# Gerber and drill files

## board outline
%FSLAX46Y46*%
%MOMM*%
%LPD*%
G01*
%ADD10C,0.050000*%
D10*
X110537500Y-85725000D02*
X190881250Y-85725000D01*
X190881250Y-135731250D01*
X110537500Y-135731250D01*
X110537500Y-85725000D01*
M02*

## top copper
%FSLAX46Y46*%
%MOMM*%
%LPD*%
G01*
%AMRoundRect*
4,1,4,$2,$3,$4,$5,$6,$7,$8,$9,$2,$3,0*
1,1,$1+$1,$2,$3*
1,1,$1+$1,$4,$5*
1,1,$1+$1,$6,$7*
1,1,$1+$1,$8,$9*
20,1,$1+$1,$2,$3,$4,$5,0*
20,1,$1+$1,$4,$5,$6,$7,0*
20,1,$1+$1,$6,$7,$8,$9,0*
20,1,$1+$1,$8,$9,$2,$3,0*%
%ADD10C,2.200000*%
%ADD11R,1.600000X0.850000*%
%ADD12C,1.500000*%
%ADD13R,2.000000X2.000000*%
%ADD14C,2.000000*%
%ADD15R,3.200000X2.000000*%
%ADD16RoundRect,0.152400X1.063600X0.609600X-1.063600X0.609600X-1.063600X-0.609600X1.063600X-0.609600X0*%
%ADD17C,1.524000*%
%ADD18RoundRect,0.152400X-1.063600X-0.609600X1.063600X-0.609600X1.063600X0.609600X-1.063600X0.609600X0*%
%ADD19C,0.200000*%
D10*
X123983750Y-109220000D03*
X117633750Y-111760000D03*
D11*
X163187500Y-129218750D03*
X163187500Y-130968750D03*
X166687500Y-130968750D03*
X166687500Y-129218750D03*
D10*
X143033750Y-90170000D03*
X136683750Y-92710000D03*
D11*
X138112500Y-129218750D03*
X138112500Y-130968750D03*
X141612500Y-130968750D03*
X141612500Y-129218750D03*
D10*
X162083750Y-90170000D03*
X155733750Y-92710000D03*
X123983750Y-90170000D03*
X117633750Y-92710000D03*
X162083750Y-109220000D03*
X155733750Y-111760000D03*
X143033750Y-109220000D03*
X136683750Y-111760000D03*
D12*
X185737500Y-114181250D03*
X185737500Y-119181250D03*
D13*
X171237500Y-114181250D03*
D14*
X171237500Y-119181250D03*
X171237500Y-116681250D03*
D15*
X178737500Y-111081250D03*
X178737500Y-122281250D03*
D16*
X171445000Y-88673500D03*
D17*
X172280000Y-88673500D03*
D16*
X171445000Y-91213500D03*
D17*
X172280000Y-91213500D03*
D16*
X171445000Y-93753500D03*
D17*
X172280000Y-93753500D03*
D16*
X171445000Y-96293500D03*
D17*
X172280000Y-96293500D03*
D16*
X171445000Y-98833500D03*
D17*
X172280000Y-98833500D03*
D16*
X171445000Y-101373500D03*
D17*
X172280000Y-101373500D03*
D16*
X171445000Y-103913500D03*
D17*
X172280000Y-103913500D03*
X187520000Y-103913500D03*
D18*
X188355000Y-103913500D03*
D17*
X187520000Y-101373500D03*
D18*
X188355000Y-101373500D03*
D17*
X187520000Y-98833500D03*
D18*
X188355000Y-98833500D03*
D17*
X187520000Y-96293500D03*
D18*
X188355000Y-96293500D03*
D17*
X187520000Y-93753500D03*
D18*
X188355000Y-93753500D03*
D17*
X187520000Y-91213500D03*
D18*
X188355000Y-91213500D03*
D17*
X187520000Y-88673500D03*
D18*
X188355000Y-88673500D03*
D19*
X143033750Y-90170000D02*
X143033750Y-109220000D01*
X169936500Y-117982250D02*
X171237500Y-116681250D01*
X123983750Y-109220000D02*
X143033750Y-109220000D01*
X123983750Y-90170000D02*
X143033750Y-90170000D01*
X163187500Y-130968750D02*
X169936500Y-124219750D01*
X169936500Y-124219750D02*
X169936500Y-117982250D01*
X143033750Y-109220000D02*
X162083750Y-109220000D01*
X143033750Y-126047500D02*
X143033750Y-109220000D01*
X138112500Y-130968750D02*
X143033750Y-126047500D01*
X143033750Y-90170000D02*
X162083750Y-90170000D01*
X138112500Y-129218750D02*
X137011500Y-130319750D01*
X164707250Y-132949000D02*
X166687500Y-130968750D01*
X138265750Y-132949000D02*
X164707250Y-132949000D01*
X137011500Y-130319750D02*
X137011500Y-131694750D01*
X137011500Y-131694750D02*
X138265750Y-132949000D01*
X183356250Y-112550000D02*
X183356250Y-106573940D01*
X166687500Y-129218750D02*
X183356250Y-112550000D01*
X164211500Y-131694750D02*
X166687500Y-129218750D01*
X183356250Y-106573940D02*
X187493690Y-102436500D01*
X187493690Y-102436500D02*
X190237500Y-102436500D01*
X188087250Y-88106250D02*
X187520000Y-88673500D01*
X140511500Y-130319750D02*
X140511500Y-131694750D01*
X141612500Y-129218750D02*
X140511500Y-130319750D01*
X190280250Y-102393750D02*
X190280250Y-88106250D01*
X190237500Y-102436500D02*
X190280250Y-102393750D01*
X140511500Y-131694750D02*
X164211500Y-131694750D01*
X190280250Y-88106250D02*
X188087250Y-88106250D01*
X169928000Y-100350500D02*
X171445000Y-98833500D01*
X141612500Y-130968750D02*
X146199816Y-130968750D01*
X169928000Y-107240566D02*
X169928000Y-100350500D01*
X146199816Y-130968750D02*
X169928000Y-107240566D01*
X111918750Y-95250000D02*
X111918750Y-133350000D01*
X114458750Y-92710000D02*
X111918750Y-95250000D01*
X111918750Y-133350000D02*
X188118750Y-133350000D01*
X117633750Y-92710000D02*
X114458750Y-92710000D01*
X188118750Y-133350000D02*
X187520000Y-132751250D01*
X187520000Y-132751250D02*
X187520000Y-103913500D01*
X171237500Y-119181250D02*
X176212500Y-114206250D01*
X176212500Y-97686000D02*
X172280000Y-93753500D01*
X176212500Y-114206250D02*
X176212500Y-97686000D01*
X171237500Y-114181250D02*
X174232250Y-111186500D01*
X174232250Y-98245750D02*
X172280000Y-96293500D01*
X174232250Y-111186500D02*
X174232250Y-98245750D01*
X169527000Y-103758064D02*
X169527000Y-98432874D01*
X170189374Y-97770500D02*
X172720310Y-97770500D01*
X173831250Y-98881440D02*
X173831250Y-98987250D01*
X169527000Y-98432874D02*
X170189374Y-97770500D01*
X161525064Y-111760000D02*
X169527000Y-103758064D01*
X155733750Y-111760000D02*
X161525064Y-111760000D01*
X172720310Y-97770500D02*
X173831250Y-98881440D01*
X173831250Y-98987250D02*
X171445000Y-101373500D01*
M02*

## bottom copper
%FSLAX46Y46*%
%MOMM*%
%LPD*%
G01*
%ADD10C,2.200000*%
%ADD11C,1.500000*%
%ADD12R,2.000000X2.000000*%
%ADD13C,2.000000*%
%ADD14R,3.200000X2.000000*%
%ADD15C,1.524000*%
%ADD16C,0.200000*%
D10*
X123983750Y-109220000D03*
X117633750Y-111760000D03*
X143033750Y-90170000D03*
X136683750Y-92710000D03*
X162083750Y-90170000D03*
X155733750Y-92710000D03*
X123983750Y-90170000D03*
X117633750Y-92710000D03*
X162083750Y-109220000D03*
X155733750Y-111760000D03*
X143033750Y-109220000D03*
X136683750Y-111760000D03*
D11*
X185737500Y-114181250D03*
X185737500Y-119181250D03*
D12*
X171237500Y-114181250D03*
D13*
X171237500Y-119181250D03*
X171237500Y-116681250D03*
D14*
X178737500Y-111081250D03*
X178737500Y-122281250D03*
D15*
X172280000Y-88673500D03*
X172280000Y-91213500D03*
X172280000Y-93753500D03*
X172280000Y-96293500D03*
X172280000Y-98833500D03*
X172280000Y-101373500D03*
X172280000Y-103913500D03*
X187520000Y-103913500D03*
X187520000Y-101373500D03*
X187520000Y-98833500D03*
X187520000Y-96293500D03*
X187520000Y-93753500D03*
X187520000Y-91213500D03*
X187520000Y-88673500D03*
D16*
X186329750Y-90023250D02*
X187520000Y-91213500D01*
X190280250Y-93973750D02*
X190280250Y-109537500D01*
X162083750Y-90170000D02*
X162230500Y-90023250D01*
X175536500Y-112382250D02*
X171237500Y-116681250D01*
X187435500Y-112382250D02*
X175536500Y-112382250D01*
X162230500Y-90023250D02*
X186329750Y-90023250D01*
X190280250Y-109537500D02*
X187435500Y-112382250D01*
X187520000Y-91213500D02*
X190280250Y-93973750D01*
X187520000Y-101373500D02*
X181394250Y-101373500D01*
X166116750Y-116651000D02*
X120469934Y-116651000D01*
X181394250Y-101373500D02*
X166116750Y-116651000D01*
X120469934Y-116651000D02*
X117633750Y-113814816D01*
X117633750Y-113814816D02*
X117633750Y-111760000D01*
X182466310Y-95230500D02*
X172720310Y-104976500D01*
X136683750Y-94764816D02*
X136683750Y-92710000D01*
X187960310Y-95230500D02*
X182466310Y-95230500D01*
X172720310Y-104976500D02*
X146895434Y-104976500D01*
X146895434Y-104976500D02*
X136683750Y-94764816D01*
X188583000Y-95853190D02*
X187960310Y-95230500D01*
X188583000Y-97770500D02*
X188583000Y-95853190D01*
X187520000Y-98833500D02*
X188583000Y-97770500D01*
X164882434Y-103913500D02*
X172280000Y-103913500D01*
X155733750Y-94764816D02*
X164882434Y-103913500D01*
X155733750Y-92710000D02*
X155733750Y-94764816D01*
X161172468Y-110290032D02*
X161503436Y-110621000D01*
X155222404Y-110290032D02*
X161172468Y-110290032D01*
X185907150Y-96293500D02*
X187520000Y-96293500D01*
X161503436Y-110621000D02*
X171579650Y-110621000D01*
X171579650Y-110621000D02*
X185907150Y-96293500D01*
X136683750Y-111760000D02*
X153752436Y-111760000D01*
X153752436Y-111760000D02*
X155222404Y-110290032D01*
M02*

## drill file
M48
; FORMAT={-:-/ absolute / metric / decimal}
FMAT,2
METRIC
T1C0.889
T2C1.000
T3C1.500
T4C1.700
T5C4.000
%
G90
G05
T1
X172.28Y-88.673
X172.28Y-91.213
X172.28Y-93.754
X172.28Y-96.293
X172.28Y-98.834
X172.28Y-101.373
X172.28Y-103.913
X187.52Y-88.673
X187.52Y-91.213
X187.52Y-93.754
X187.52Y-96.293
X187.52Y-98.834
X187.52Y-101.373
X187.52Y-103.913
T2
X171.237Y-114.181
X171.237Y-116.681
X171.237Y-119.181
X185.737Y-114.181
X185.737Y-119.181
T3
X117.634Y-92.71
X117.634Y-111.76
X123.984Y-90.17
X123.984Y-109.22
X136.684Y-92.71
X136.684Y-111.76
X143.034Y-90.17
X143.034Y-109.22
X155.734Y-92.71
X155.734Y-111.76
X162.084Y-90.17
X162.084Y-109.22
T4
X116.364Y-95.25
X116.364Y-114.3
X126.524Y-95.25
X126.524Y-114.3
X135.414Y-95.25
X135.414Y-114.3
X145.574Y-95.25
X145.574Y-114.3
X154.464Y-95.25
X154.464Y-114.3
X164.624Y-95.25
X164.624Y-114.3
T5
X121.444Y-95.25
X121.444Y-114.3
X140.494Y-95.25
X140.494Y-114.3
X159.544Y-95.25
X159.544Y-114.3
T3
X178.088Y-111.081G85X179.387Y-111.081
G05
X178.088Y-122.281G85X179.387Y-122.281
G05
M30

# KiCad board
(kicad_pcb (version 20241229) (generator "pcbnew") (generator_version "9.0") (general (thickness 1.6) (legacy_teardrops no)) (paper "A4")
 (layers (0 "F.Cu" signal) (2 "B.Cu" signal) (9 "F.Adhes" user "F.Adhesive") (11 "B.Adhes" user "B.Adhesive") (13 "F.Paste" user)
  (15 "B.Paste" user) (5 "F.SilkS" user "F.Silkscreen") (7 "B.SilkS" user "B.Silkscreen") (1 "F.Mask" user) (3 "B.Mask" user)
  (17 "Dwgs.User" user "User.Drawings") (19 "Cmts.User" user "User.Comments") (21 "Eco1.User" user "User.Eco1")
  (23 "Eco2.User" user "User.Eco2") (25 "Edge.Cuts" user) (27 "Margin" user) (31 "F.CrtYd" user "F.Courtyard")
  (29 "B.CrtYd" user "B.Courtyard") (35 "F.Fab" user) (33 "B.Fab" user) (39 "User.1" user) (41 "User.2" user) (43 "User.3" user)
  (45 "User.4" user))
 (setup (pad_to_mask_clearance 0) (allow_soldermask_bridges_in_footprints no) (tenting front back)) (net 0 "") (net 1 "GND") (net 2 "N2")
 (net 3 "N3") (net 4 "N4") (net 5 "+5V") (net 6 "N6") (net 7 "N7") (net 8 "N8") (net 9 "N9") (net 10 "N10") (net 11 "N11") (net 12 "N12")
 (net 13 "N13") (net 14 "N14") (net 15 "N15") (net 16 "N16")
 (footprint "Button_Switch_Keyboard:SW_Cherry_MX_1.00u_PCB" (layer "F.Cu") (at 123.98375 109.22)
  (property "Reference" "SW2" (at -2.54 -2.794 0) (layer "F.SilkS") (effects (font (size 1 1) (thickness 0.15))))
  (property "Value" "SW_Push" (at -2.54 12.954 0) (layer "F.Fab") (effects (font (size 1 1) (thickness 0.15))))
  (pad "" np_thru_hole circle (at -7.62 5.08) (size 1.7 1.7) (drill 1.7) (layers "*.Cu" "*.Mask"))
  (pad "" np_thru_hole circle (at -2.54 5.08) (size 4 4) (drill 4) (layers "*.Cu" "*.Mask"))
  (pad "" np_thru_hole circle (at 2.54 5.08) (size 1.7 1.7) (drill 1.7) (layers "*.Cu" "*.Mask"))
  (pad "1" thru_hole circle (at 0 0) (size 2.2 2.2) (drill 1.5) (layers "*.Cu" "*.Mask") (remove_unused_layers no) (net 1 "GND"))
  (pad "2" thru_hole circle (at -6.35 2.54) (size 2.2 2.2) (drill 1.5) (layers "*.Cu" "*.Mask") (remove_unused_layers no) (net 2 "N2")))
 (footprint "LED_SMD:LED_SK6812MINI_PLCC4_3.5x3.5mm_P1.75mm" (layer "F.Cu") (at 164.9375 130.09375)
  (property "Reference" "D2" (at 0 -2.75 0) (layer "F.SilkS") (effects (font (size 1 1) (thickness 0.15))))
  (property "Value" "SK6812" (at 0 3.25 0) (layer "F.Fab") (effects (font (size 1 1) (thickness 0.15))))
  (pad "1" smd rect (at -1.75 -0.875) (size 1.6 0.85) (layers "F.Cu" "F.Mask" "F.Paste") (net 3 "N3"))
  (pad "2" smd rect (at -1.75 0.875) (size 1.6 0.85) (layers "F.Cu" "F.Mask" "F.Paste") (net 1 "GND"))
  (pad "3" smd rect (at 1.75 0.875) (size 1.6 0.85) (layers "F.Cu" "F.Mask" "F.Paste") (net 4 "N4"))
  (pad "4" smd rect (at 1.75 -0.875) (size 1.6 0.85) (layers "F.Cu" "F.Mask" "F.Paste") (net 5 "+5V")))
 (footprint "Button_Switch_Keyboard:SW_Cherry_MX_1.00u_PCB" (layer "F.Cu") (at 143.03375 90.17)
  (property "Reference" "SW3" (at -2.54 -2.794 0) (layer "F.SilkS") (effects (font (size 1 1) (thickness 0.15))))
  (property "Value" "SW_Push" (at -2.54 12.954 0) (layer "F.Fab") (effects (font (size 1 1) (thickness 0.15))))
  (pad "" np_thru_hole circle (at -7.62 5.08) (size 1.7 1.7) (drill 1.7) (layers "*.Cu" "*.Mask"))
  (pad "" np_thru_hole circle (at -2.54 5.08) (size 4 4) (drill 4) (layers "*.Cu" "*.Mask"))
  (pad "" np_thru_hole circle (at 2.54 5.08) (size 1.7 1.7) (drill 1.7) (layers "*.Cu" "*.Mask"))
  (pad "1" thru_hole circle (at 0 0) (size 2.2 2.2) (drill 1.5) (layers "*.Cu" "*.Mask") (remove_unused_layers no) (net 1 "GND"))
  (pad "2" thru_hole circle (at -6.35 2.54) (size 2.2 2.2) (drill 1.5) (layers "*.Cu" "*.Mask") (remove_unused_layers no) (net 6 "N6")))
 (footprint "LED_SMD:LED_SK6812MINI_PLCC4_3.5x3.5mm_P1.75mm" (layer "F.Cu") (at 139.8625 130.09375)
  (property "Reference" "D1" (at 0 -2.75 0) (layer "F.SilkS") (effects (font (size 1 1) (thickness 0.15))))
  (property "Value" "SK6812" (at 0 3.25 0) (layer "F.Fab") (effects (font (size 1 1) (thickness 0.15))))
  (pad "1" smd rect (at -1.75 -0.875) (size 1.6 0.85) (layers "F.Cu" "F.Mask" "F.Paste") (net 4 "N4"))
  (pad "2" smd rect (at -1.75 0.875) (size 1.6 0.85) (layers "F.Cu" "F.Mask" "F.Paste") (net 1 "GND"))
  (pad "3" smd rect (at 1.75 0.875) (size 1.6 0.85) (layers "F.Cu" "F.Mask" "F.Paste") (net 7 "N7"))
  (pad "4" smd rect (at 1.75 -0.875) (size 1.6 0.85) (layers "F.Cu" "F.Mask" "F.Paste") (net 5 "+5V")))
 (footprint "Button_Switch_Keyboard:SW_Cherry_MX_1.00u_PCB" (layer "F.Cu") (at 162.08375 90.17)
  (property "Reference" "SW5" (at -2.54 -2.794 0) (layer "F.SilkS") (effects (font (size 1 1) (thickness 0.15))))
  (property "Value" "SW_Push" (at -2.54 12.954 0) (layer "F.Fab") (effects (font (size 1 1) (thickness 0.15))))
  (pad "" np_thru_hole circle (at -7.62 5.08) (size 1.7 1.7) (drill 1.7) (layers "*.Cu" "*.Mask"))
  (pad "" np_thru_hole circle (at -2.54 5.08) (size 4 4) (drill 4) (layers "*.Cu" "*.Mask"))
  (pad "" np_thru_hole circle (at 2.54 5.08) (size 1.7 1.7) (drill 1.7) (layers "*.Cu" "*.Mask"))
  (pad "1" thru_hole circle (at 0 0) (size 2.2 2.2) (drill 1.5) (layers "*.Cu" "*.Mask") (remove_unused_layers no) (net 1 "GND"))
  (pad "2" thru_hole circle (at -6.35 2.54) (size 2.2 2.2) (drill 1.5) (layers "*.Cu" "*.Mask") (remove_unused_layers no) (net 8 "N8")))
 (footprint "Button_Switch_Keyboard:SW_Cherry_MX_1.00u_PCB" (layer "F.Cu") (at 123.98375 90.17)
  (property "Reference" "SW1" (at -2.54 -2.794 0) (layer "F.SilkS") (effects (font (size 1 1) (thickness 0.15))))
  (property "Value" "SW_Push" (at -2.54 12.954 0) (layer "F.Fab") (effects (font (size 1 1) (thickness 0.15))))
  (pad "" np_thru_hole circle (at -7.62 5.08) (size 1.7 1.7) (drill 1.7) (layers "*.Cu" "*.Mask"))
  (pad "" np_thru_hole circle (at -2.54 5.08) (size 4 4) (drill 4) (layers "*.Cu" "*.Mask"))
  (pad "" np_thru_hole circle (at 2.54 5.08) (size 1.7 1.7) (drill 1.7) (layers "*.Cu" "*.Mask"))
  (pad "1" thru_hole circle (at 0 0) (size 2.2 2.2) (drill 1.5) (layers "*.Cu" "*.Mask") (remove_unused_layers no) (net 1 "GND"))
  (pad "2" thru_hole circle (at -6.35 2.54) (size 2.2 2.2) (drill 1.5) (layers "*.Cu" "*.Mask") (remove_unused_layers no) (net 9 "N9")))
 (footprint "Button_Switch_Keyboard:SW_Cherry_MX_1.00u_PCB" (layer "F.Cu") (at 162.08375 109.22)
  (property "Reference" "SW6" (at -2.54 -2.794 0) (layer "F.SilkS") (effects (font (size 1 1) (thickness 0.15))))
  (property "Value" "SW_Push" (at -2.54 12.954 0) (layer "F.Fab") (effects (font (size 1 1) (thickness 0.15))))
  (pad "" np_thru_hole circle (at -7.62 5.08) (size 1.7 1.7) (drill 1.7) (layers "*.Cu" "*.Mask"))
  (pad "" np_thru_hole circle (at -2.54 5.08) (size 4 4) (drill 4) (layers "*.Cu" "*.Mask"))
  (pad "" np_thru_hole circle (at 2.54 5.08) (size 1.7 1.7) (drill 1.7) (layers "*.Cu" "*.Mask"))
  (pad "1" thru_hole circle (at 0 0) (size 2.2 2.2) (drill 1.5) (layers "*.Cu" "*.Mask") (remove_unused_layers no) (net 1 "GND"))
  (pad "2" thru_hole circle (at -6.35 2.54) (size 2.2 2.2) (drill 1.5) (layers "*.Cu" "*.Mask") (remove_unused_layers no) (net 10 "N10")))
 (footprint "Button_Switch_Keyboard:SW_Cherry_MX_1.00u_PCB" (layer "F.Cu") (at 143.03375 109.22)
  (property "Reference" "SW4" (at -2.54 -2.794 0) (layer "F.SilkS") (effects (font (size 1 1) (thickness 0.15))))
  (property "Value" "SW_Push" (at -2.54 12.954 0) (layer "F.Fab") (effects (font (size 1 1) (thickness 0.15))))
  (pad "" np_thru_hole circle (at -7.62 5.08) (size 1.7 1.7) (drill 1.7) (layers "*.Cu" "*.Mask"))
  (pad "" np_thru_hole circle (at -2.54 5.08) (size 4 4) (drill 4) (layers "*.Cu" "*.Mask"))
  (pad "" np_thru_hole circle (at 2.54 5.08) (size 1.7 1.7) (drill 1.7) (layers "*.Cu" "*.Mask"))
  (pad "1" thru_hole circle (at 0 0) (size 2.2 2.2) (drill 1.5) (layers "*.Cu" "*.Mask") (remove_unused_layers no) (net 1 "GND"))
  (pad "2" thru_hole circle (at -6.35 2.54) (size 2.2 2.2) (drill 1.5) (layers "*.Cu" "*.Mask") (remove_unused_layers no) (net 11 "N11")))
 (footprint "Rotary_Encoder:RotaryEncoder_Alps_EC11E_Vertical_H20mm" (layer "F.Cu") (at 171.2375 114.18125)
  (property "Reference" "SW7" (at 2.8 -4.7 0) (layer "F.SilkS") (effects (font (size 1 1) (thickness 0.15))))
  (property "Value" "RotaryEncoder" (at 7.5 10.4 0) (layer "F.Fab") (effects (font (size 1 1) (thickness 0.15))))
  (pad "" thru_hole circle (at 14.5 0) (size 1.5 1.5) (drill 1) (layers "*.Cu" "*.Mask") (remove_unused_layers no))
  (pad "" thru_hole circle (at 14.5 5) (size 1.5 1.5) (drill 1) (layers "*.Cu" "*.Mask") (remove_unused_layers no))
  (pad "A" thru_hole rect (at 0 0) (size 2 2) (drill 1) (layers "*.Cu" "*.Mask") (remove_unused_layers no) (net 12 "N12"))
  (pad "B" thru_hole circle (at 0 5) (size 2 2) (drill 1) (layers "*.Cu" "*.Mask") (remove_unused_layers no) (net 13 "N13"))
  (pad "C" thru_hole circle (at 0 2.5) (size 2 2) (drill 1) (layers "*.Cu" "*.Mask") (remove_unused_layers no) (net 1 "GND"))
  (pad "MP" thru_hole rect (at 7.5 -3.1) (size 3.2 2) (drill oval 2.8 1.5) (layers "*.Cu" "*.Mask") (remove_unused_layers no))
  (pad "MP" thru_hole rect (at 7.5 8.1) (size 3.2 2) (drill oval 2.8 1.5) (layers "*.Cu" "*.Mask") (remove_unused_layers no)))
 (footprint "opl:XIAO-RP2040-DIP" (layer "F.Cu") (at 179.9 96.2935)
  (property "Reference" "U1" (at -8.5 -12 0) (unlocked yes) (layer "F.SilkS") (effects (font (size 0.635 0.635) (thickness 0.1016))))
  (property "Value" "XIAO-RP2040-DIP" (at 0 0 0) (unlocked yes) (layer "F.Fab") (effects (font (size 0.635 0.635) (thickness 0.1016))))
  (pad "1" smd roundrect (at -8.455 -7.62 180) (size 2.432 1.524) (layers "F.Cu" "F.Mask") (roundrect_rratio 0.1) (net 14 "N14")
   (thermal_bridge_angle 45))
  (pad "1" thru_hole circle (at -7.62 -7.62 180) (size 1.524 1.524) (drill 0.889) (layers "*.Cu" "*.Mask") (remove_unused_layers no)
   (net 14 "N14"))
  (pad "2" smd roundrect (at -8.455 -5.08 180) (size 2.432 1.524) (layers "F.Cu" "F.Mask") (roundrect_rratio 0.1) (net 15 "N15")
   (thermal_bridge_angle 45))
  (pad "2" thru_hole circle (at -7.62 -5.08 180) (size 1.524 1.524) (drill 0.889) (layers "*.Cu" "*.Mask") (remove_unused_layers no)
   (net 15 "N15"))
  (pad "3" smd roundrect (at -8.455 -2.54 180) (size 2.432 1.524) (layers "F.Cu" "F.Mask") (roundrect_rratio 0.1) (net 13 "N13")
   (thermal_bridge_angle 45))
  (pad "3" thru_hole circle (at -7.62 -2.54 180) (size 1.524 1.524) (drill 0.889) (layers "*.Cu" "*.Mask") (remove_unused_layers no)
   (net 13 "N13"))
  (pad "4" smd roundrect (at -8.455 0 180) (size 2.432 1.524) (layers "F.Cu" "F.Mask") (roundrect_rratio 0.1) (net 12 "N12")
   (thermal_bridge_angle 45))
  (pad "4" thru_hole circle (at -7.62 0 180) (size 1.524 1.524) (drill 0.889) (layers "*.Cu" "*.Mask") (remove_unused_layers no)
   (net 12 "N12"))
  (pad "5" smd roundrect (at -8.455 2.54 180) (size 2.432 1.524) (layers "F.Cu" "F.Mask") (roundrect_rratio 0.1) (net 7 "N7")
   (thermal_bridge_angle 45))
  (pad "5" thru_hole circle (at -7.62 2.54 180) (size 1.524 1.524) (drill 0.889) (layers "*.Cu" "*.Mask") (remove_unused_layers no)
   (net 7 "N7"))
  (pad "6" smd roundrect (at -8.455 5.08 180) (size 2.432 1.524) (layers "F.Cu" "F.Mask") (roundrect_rratio 0.1) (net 10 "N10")
   (thermal_bridge_angle 45))
  (pad "6" thru_hole circle (at -7.62 5.08 180) (size 1.524 1.524) (drill 0.889) (layers "*.Cu" "*.Mask") (remove_unused_layers no)
   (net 10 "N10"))
  (pad "7" smd roundrect (at -8.455 7.62 180) (size 2.432 1.524) (layers "F.Cu" "F.Mask") (roundrect_rratio 0.1) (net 8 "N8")
   (thermal_bridge_angle 45))
  (pad "7" thru_hole circle (at -7.62 7.62 180) (size 1.524 1.524) (drill 0.889) (layers "*.Cu" "*.Mask") (remove_unused_layers no)
   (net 8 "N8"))
  (pad "8" thru_hole circle (at 7.62 7.62) (size 1.524 1.524) (drill 0.889) (layers "*.Cu" "*.Mask") (remove_unused_layers no) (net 9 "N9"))
  (pad "8" smd roundrect (at 8.455 7.62) (size 2.432 1.524) (layers "F.Cu" "F.Mask") (roundrect_rratio 0.1) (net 9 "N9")
   (thermal_bridge_angle 45))
  (pad "9" thru_hole circle (at 7.62 5.08) (size 1.524 1.524) (drill 0.889) (layers "*.Cu" "*.Mask") (remove_unused_layers no) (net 2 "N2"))
  (pad "9" smd roundrect (at 8.455 5.08) (size 2.432 1.524) (layers "F.Cu" "F.Mask") (roundrect_rratio 0.1) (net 2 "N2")
   (thermal_bridge_angle 45))
  (pad "10" thru_hole circle (at 7.62 2.54) (size 1.524 1.524) (drill 0.889) (layers "*.Cu" "*.Mask") (remove_unused_layers no) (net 6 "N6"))
  (pad "10" smd roundrect (at 8.455 2.54) (size 2.432 1.524) (layers "F.Cu" "F.Mask") (roundrect_rratio 0.1) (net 6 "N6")
   (thermal_bridge_angle 45))
  (pad "11" thru_hole circle (at 7.62 0) (size 1.524 1.524) (drill 0.889) (layers "*.Cu" "*.Mask") (remove_unused_layers no) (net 11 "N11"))
  (pad "11" smd roundrect (at 8.455 0) (size 2.432 1.524) (layers "F.Cu" "F.Mask") (roundrect_rratio 0.1) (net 11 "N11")
   (thermal_bridge_angle 45))
  (pad "12" thru_hole circle (at 7.62 -2.54) (size 1.524 1.524) (drill 0.889) (layers "*.Cu" "*.Mask") (remove_unused_layers no)
   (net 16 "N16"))
  (pad "12" smd roundrect (at 8.455 -2.54) (size 2.432 1.524) (layers "F.Cu" "F.Mask") (roundrect_rratio 0.1) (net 16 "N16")
   (thermal_bridge_angle 45))
  (pad "13" thru_hole circle (at 7.62 -5.08) (size 1.524 1.524) (drill 0.889) (layers "*.Cu" "*.Mask") (remove_unused_layers no)
   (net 1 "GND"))
  (pad "13" smd roundrect (at 8.455 -5.08) (size 2.432 1.524) (layers "F.Cu" "F.Mask") (roundrect_rratio 0.1) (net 1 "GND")
   (thermal_bridge_angle 45))
  (pad "14" thru_hole circle (at 7.62 -7.62) (size 1.524 1.524) (drill 0.889) (layers "*.Cu" "*.Mask") (remove_unused_layers no)
   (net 5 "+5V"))
  (pad "14" smd roundrect (at 8.455 -7.62) (size 2.432 1.524) (layers "F.Cu" "F.Mask") (roundrect_rratio 0.1) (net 5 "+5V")
   (thermal_bridge_angle 45)))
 (gr_rect (start 110.5375 85.725) (end 190.88125 135.73125) (stroke (width 0.05) (type default)) (fill no) (layer "Edge.Cuts"))
 (segment (start 143.03375 90.17) (end 143.03375 109.22) (width 0.2) (layer "F.Cu") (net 1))
 (segment (start 169.9365 117.98225) (end 171.2375 116.68125) (width 0.2) (layer "F.Cu") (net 1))
 (segment (start 123.98375 109.22) (end 143.03375 109.22) (width 0.2) (layer "F.Cu") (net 1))
 (segment (start 123.98375 90.17) (end 143.03375 90.17) (width 0.2) (layer "F.Cu") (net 1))
 (segment (start 163.1875 130.96875) (end 169.9365 124.21975) (width 0.2) (layer "F.Cu") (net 1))
 (segment (start 169.9365 124.21975) (end 169.9365 117.98225) (width 0.2) (layer "F.Cu") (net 1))
 (segment (start 143.03375 109.22) (end 162.08375 109.22) (width 0.2) (layer "F.Cu") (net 1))
 (segment (start 143.03375 126.0475) (end 143.03375 109.22) (width 0.2) (layer "F.Cu") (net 1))
 (segment (start 138.1125 130.96875) (end 143.03375 126.0475) (width 0.2) (layer "F.Cu") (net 1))
 (segment (start 143.03375 90.17) (end 162.08375 90.17) (width 0.2) (layer "F.Cu") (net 1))
 (segment (start 186.32975 90.02325) (end 187.52 91.2135) (width 0.2) (layer "B.Cu") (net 1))
 (segment (start 190.28025 93.97375) (end 190.28025 109.5375) (width 0.2) (layer "B.Cu") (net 1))
 (segment (start 162.08375 90.17) (end 162.2305 90.02325) (width 0.2) (layer "B.Cu") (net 1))
 (segment (start 175.5365 112.38225) (end 171.2375 116.68125) (width 0.2) (layer "B.Cu") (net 1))
 (segment (start 187.4355 112.38225) (end 175.5365 112.38225) (width 0.2) (layer "B.Cu") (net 1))
 (segment (start 162.2305 90.02325) (end 186.32975 90.02325) (width 0.2) (layer "B.Cu") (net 1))
 (segment (start 190.28025 109.5375) (end 187.4355 112.38225) (width 0.2) (layer "B.Cu") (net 1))
 (segment (start 187.52 91.2135) (end 190.28025 93.97375) (width 0.2) (layer "B.Cu") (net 1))
 (segment (start 138.1125 129.21875) (end 137.0115 130.31975) (width 0.2) (layer "F.Cu") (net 4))
 (segment (start 164.70725 132.949) (end 166.6875 130.96875) (width 0.2) (layer "F.Cu") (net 4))
 (segment (start 138.26575 132.949) (end 164.70725 132.949) (width 0.2) (layer "F.Cu") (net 4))
 (segment (start 137.0115 130.31975) (end 137.0115 131.69475) (width 0.2) (layer "F.Cu") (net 4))
 (segment (start 137.0115 131.69475) (end 138.26575 132.949) (width 0.2) (layer "F.Cu") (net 4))
 (segment (start 183.35625 112.55) (end 183.35625 106.57394) (width 0.2) (layer "F.Cu") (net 5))
 (segment (start 166.6875 129.21875) (end 183.35625 112.55) (width 0.2) (layer "F.Cu") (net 5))
 (segment (start 164.2115 131.69475) (end 166.6875 129.21875) (width 0.2) (layer "F.Cu") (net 5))
 (segment (start 183.35625 106.57394) (end 187.49369 102.4365) (width 0.2) (layer "F.Cu") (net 5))
 (segment (start 187.49369 102.4365) (end 190.2375 102.4365) (width 0.2) (layer "F.Cu") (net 5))
 (segment (start 188.08725 88.10625) (end 187.52 88.6735) (width 0.2) (layer "F.Cu") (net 5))
 (segment (start 140.5115 130.31975) (end 140.5115 131.69475) (width 0.2) (layer "F.Cu") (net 5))
 (segment (start 141.6125 129.21875) (end 140.5115 130.31975) (width 0.2) (layer "F.Cu") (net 5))
 (segment (start 190.28025 102.39375) (end 190.28025 88.10625) (width 0.2) (layer "F.Cu") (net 5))
 (segment (start 190.2375 102.4365) (end 190.28025 102.39375) (width 0.2) (layer "F.Cu") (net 5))
 (segment (start 140.5115 131.69475) (end 164.2115 131.69475) (width 0.2) (layer "F.Cu") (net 5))
 (segment (start 190.28025 88.10625) (end 188.08725 88.10625) (width 0.2) (layer "F.Cu") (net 5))
 (segment (start 169.928 100.3505) (end 171.445 98.8335) (width 0.2) (layer "F.Cu") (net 7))
 (segment (start 141.6125 130.96875) (end 146.199816 130.96875) (width 0.2) (layer "F.Cu") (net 7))
 (segment (start 169.928 107.240566) (end 169.928 100.3505) (width 0.2) (layer "F.Cu") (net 7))
 (segment (start 146.199816 130.96875) (end 169.928 107.240566) (width 0.2) (layer "F.Cu") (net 7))
 (segment (start 111.91875 95.25) (end 111.91875 133.35) (width 0.2) (layer "F.Cu") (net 9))
 (segment (start 114.45875 92.71) (end 111.91875 95.25) (width 0.2) (layer "F.Cu") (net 9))
 (segment (start 111.91875 133.35) (end 188.11875 133.35) (width 0.2) (layer "F.Cu") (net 9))
 (segment (start 117.63375 92.71) (end 114.45875 92.71) (width 0.2) (layer "F.Cu") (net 9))
 (segment (start 188.11875 133.35) (end 187.52 132.75125) (width 0.2) (layer "F.Cu") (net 9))
 (segment (start 187.52 132.75125) (end 187.52 103.9135) (width 0.2) (layer "F.Cu") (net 9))
 (segment (start 187.52 101.3735) (end 181.39425 101.3735) (width 0.2) (layer "B.Cu") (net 2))
 (segment (start 166.11675 116.651) (end 120.469934 116.651) (width 0.2) (layer "B.Cu") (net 2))
 (segment (start 181.39425 101.3735) (end 166.11675 116.651) (width 0.2) (layer "B.Cu") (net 2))
 (segment (start 120.469934 116.651) (end 117.63375 113.814816) (width 0.2) (layer "B.Cu") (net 2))
 (segment (start 117.63375 113.814816) (end 117.63375 111.76) (width 0.2) (layer "B.Cu") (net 2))
 (segment (start 182.46631 95.2305) (end 172.72031 104.9765) (width 0.2) (layer "B.Cu") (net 6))
 (segment (start 136.68375 94.764816) (end 136.68375 92.71) (width 0.2) (layer "B.Cu") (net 6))
 (segment (start 187.96031 95.2305) (end 182.46631 95.2305) (width 0.2) (layer "B.Cu") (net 6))
 (segment (start 172.72031 104.9765) (end 146.895434 104.9765) (width 0.2) (layer "B.Cu") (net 6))
 (segment (start 146.895434 104.9765) (end 136.68375 94.764816) (width 0.2) (layer "B.Cu") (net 6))
 (segment (start 188.583 95.85319) (end 187.96031 95.2305) (width 0.2) (layer "B.Cu") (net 6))
 (segment (start 188.583 97.7705) (end 188.583 95.85319) (width 0.2) (layer "B.Cu") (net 6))
 (segment (start 187.52 98.8335) (end 188.583 97.7705) (width 0.2) (layer "B.Cu") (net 6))
 (segment (start 171.2375 119.18125) (end 176.2125 114.20625) (width 0.2) (layer "F.Cu") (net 13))
 (segment (start 176.2125 97.686) (end 172.28 93.7535) (width 0.2) (layer "F.Cu") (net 13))
 (segment (start 176.2125 114.20625) (end 176.2125 97.686) (width 0.2) (layer "F.Cu") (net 13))
 (segment (start 171.2375 114.18125) (end 174.23225 111.1865) (width 0.2) (layer "F.Cu") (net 12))
 (segment (start 174.23225 98.24575) (end 172.28 96.2935) (width 0.2) (layer "F.Cu") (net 12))
 (segment (start 174.23225 111.1865) (end 174.23225 98.24575) (width 0.2) (layer "F.Cu") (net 12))
 (segment (start 164.882434 103.9135) (end 172.28 103.9135) (width 0.2) (layer "B.Cu") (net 8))
 (segment (start 155.73375 94.764816) (end 164.882434 103.9135) (width 0.2) (layer "B.Cu") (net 8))
 (segment (start 155.73375 92.71) (end 155.73375 94.764816) (width 0.2) (layer "B.Cu") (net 8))
 (segment (start 169.527 103.758064) (end 169.527 98.432874) (width 0.2) (layer "F.Cu") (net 10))
 (segment (start 170.189374 97.7705) (end 172.72031 97.7705) (width 0.2) (layer "F.Cu") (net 10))
 (segment (start 173.83125 98.88144) (end 173.83125 98.98725) (width 0.2) (layer "F.Cu") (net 10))
 (segment (start 169.527 98.432874) (end 170.189374 97.7705) (width 0.2) (layer "F.Cu") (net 10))
 (segment (start 161.525064 111.76) (end 169.527 103.758064) (width 0.2) (layer "F.Cu") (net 10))
 (segment (start 155.73375 111.76) (end 161.525064 111.76) (width 0.2) (layer "F.Cu") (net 10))
 (segment (start 172.72031 97.7705) (end 173.83125 98.88144) (width 0.2) (layer "F.Cu") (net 10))
 (segment (start 173.83125 98.98725) (end 171.445 101.3735) (width 0.2) (layer "F.Cu") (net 10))
 (segment (start 161.172468 110.290032) (end 161.503436 110.621) (width 0.2) (layer "B.Cu") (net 11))
 (segment (start 155.222404 110.290032) (end 161.172468 110.290032) (width 0.2) (layer "B.Cu") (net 11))
 (segment (start 185.90715 96.2935) (end 187.52 96.2935) (width 0.2) (layer "B.Cu") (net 11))
 (segment (start 161.503436 110.621) (end 171.57965 110.621) (width 0.2) (layer "B.Cu") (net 11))
 (segment (start 171.57965 110.621) (end 185.90715 96.2935) (width 0.2) (layer "B.Cu") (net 11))
 (segment (start 136.68375 111.76) (end 153.752436 111.76) (width 0.2) (layer "B.Cu") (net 11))
 (segment (start 153.752436 111.76) (end 155.222404 110.290032) (width 0.2) (layer "B.Cu") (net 11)))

